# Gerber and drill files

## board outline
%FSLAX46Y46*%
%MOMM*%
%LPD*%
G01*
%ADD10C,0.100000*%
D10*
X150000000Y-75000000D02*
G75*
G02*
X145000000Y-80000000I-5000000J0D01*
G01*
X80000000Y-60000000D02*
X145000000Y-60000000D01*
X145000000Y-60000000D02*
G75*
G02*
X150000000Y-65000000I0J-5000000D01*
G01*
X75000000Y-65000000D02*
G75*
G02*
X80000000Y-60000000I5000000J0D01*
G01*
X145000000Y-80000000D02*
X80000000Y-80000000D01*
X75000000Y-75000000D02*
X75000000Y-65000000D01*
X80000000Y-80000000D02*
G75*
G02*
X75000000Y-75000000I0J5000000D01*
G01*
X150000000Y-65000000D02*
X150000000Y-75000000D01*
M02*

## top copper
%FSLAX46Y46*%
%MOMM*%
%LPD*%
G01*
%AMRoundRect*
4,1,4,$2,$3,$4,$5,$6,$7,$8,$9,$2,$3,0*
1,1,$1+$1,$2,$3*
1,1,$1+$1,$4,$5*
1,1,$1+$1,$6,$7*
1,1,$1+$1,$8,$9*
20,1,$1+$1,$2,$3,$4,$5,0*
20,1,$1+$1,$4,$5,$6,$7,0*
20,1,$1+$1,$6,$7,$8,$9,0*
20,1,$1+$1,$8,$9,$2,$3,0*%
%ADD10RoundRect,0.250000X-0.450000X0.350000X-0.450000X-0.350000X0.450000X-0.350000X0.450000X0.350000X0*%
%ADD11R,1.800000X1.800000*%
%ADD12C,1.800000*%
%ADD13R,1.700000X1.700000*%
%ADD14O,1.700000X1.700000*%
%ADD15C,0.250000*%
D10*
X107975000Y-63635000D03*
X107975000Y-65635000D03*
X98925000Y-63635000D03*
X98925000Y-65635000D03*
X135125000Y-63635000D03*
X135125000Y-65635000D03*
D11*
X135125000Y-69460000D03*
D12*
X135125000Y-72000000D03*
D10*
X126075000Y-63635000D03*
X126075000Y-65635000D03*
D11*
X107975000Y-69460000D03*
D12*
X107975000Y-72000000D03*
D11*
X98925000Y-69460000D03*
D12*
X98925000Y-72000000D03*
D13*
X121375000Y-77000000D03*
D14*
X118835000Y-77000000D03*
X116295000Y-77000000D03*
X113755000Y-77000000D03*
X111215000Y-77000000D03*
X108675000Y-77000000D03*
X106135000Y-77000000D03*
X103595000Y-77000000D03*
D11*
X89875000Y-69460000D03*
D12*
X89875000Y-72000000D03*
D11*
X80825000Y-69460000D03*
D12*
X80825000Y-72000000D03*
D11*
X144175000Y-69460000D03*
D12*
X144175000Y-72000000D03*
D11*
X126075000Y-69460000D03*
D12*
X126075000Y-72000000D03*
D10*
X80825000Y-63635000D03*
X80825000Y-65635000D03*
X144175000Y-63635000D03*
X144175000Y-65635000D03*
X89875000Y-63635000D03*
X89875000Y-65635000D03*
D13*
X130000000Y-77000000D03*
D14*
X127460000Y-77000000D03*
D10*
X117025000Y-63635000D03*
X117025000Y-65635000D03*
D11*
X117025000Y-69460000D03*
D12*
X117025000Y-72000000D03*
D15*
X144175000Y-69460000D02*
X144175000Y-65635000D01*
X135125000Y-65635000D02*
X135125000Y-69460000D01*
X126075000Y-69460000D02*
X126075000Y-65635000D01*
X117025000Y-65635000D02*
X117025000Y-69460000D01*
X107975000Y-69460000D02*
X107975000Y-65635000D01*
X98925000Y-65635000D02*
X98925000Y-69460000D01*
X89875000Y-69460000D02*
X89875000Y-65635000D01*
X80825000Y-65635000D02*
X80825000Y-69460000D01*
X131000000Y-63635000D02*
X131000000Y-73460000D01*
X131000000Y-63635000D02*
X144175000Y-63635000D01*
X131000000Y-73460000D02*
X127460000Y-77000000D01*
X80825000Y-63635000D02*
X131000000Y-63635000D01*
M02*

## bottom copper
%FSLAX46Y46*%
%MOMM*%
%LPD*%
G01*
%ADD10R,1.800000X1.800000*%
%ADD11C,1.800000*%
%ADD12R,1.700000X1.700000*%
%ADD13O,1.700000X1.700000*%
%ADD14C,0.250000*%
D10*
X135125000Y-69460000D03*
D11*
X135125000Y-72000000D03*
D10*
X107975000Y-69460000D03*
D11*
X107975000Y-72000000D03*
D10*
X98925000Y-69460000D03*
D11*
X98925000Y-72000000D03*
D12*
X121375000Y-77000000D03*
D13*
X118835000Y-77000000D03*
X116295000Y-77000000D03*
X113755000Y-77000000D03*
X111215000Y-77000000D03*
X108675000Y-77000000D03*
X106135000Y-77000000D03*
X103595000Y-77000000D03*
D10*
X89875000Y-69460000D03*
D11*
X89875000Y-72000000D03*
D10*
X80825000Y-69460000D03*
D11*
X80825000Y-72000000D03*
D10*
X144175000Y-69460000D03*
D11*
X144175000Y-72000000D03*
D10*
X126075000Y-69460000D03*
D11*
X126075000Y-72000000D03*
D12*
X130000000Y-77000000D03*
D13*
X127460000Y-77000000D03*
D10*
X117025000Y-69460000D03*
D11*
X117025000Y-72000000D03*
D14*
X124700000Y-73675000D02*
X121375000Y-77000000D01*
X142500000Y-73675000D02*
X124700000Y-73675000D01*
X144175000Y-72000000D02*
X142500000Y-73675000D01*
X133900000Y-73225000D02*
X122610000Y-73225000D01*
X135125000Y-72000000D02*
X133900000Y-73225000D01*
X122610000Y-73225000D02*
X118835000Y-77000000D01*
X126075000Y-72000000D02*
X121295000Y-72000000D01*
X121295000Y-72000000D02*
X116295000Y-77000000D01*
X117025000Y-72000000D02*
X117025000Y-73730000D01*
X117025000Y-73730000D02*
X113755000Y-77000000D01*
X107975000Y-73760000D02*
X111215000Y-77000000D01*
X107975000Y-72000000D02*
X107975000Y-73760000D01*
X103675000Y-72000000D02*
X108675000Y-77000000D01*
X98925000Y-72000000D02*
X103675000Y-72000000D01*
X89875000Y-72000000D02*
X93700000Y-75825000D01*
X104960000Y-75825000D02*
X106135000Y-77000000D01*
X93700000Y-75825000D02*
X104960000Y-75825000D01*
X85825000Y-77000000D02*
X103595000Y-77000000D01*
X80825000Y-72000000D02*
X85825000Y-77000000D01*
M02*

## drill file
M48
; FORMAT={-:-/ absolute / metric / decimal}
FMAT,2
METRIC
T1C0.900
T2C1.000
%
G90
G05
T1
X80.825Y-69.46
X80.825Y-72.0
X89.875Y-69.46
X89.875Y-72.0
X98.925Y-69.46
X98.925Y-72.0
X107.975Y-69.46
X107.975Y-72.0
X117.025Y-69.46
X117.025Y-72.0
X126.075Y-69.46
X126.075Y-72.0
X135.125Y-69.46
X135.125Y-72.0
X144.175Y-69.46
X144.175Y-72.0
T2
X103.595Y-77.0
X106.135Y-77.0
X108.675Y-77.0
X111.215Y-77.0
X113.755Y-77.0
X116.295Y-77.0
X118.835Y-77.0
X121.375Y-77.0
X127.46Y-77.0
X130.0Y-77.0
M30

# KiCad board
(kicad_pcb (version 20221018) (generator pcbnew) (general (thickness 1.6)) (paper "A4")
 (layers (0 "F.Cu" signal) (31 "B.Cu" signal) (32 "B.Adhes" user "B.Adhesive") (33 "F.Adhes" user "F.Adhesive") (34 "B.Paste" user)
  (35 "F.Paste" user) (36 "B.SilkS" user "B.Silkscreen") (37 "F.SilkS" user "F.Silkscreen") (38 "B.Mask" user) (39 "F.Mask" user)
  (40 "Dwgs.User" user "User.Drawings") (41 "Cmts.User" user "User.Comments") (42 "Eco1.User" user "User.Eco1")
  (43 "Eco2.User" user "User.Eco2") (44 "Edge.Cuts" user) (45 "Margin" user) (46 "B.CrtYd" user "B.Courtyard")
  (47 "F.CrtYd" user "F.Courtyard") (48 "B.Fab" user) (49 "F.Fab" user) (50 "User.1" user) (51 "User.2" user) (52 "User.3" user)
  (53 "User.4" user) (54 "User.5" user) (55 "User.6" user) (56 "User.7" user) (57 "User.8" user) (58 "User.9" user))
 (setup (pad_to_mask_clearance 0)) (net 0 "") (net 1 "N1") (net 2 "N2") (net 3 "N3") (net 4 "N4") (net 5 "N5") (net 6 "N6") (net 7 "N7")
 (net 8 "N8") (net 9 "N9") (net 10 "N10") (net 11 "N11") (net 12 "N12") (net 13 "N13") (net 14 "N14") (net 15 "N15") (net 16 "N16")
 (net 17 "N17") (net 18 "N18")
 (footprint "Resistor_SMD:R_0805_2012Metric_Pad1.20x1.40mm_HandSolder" (layer "F.Cu") (at 107.975 64.635 -90)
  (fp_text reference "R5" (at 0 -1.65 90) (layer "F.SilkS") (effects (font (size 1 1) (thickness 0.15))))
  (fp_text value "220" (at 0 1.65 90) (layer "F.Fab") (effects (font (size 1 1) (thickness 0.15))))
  (pad "1" smd roundrect (at -1 0 270) (size 1.2 1.4) (layers "F.Cu" "F.Paste" "F.Mask") (roundrect_rratio 0.208333) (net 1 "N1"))
  (pad "2" smd roundrect (at 1 0 270) (size 1.2 1.4) (layers "F.Cu" "F.Paste" "F.Mask") (roundrect_rratio 0.208333) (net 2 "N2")))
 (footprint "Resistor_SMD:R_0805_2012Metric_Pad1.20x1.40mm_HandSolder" (layer "F.Cu") (at 98.925 64.635 -90)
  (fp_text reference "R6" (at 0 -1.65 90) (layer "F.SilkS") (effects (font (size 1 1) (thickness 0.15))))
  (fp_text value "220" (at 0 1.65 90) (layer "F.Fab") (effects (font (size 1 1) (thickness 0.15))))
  (pad "1" smd roundrect (at -1 0 270) (size 1.2 1.4) (layers "F.Cu" "F.Paste" "F.Mask") (roundrect_rratio 0.208333) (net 1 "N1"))
  (pad "2" smd roundrect (at 1 0 270) (size 1.2 1.4) (layers "F.Cu" "F.Paste" "F.Mask") (roundrect_rratio 0.208333) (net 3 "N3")))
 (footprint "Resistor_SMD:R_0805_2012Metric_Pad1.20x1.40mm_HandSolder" (layer "F.Cu") (at 135.125 64.635 -90)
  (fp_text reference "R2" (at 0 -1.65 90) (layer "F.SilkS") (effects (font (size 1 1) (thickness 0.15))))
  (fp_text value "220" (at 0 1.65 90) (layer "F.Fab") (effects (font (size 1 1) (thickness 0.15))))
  (pad "1" smd roundrect (at -1 0 270) (size 1.2 1.4) (layers "F.Cu" "F.Paste" "F.Mask") (roundrect_rratio 0.208333) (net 1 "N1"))
  (pad "2" smd roundrect (at 1 0 270) (size 1.2 1.4) (layers "F.Cu" "F.Paste" "F.Mask") (roundrect_rratio 0.208333) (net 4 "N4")))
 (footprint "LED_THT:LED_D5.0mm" (layer "F.Cu") (at 135.125 69.46 -90)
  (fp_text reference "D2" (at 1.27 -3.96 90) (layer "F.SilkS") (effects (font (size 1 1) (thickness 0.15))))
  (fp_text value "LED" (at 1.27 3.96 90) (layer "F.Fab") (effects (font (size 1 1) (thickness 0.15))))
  (pad "1" thru_hole rect (at 0 0 270) (size 1.8 1.8) (drill 0.9) (layers "*.Cu" "*.Mask") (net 4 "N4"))
  (pad "2" thru_hole circle (at 2.54 0 270) (size 1.8 1.8) (drill 0.9) (layers "*.Cu" "*.Mask") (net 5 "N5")))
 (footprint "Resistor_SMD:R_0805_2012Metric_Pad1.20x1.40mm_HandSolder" (layer "F.Cu") (at 126.075 64.635 -90)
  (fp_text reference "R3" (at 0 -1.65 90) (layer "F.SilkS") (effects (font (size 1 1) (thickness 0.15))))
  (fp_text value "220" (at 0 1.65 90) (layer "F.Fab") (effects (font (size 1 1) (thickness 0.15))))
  (pad "1" smd roundrect (at -1 0 270) (size 1.2 1.4) (layers "F.Cu" "F.Paste" "F.Mask") (roundrect_rratio 0.208333) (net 1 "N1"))
  (pad "2" smd roundrect (at 1 0 270) (size 1.2 1.4) (layers "F.Cu" "F.Paste" "F.Mask") (roundrect_rratio 0.208333) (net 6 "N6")))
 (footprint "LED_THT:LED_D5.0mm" (layer "F.Cu") (at 107.975 69.46 -90)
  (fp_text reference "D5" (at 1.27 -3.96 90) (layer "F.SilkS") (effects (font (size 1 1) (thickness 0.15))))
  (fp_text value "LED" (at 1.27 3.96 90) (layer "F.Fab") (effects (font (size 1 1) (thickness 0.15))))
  (pad "1" thru_hole rect (at 0 0 270) (size 1.8 1.8) (drill 0.9) (layers "*.Cu" "*.Mask") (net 2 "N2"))
  (pad "2" thru_hole circle (at 2.54 0 270) (size 1.8 1.8) (drill 0.9) (layers "*.Cu" "*.Mask") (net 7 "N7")))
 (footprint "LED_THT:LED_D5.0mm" (layer "F.Cu") (at 98.925 69.46 -90)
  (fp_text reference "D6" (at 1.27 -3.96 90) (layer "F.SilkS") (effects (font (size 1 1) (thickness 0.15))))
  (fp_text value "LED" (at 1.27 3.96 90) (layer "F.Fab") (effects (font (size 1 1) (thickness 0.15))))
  (pad "1" thru_hole rect (at 0 0 270) (size 1.8 1.8) (drill 0.9) (layers "*.Cu" "*.Mask") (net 3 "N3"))
  (pad "2" thru_hole circle (at 2.54 0 270) (size 1.8 1.8) (drill 0.9) (layers "*.Cu" "*.Mask") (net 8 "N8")))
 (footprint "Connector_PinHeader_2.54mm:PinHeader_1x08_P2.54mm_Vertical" (layer "F.Cu") (at 121.375 77 -90)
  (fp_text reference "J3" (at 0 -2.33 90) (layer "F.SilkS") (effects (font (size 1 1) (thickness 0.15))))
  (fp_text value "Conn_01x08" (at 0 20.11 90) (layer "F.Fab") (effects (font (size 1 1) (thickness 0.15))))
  (pad "1" thru_hole rect (at 0 0 270) (size 1.7 1.7) (drill 1) (layers "*.Cu" "*.Mask") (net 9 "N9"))
  (pad "2" thru_hole oval (at 0 2.54 270) (size 1.7 1.7) (drill 1) (layers "*.Cu" "*.Mask") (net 5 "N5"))
  (pad "3" thru_hole oval (at 0 5.08 270) (size 1.7 1.7) (drill 1) (layers "*.Cu" "*.Mask") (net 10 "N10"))
  (pad "4" thru_hole oval (at 0 7.62 270) (size 1.7 1.7) (drill 1) (layers "*.Cu" "*.Mask") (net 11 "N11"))
  (pad "5" thru_hole oval (at 0 10.16 270) (size 1.7 1.7) (drill 1) (layers "*.Cu" "*.Mask") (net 7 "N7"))
  (pad "6" thru_hole oval (at 0 12.7 270) (size 1.7 1.7) (drill 1) (layers "*.Cu" "*.Mask") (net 8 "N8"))
  (pad "7" thru_hole oval (at 0 15.24 270) (size 1.7 1.7) (drill 1) (layers "*.Cu" "*.Mask") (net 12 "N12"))
  (pad "8" thru_hole oval (at 0 17.78 270) (size 1.7 1.7) (drill 1) (layers "*.Cu" "*.Mask") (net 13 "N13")))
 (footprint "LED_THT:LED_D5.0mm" (layer "F.Cu") (at 89.875 69.46 -90)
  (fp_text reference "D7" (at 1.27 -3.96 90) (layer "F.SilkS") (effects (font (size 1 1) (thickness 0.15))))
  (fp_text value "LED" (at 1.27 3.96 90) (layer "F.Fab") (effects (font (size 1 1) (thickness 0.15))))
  (pad "1" thru_hole rect (at 0 0 270) (size 1.8 1.8) (drill 0.9) (layers "*.Cu" "*.Mask") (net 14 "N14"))
  (pad "2" thru_hole circle (at 2.54 0 270) (size 1.8 1.8) (drill 0.9) (layers "*.Cu" "*.Mask") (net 12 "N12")))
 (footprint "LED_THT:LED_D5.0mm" (layer "F.Cu") (at 80.825 69.46 -90)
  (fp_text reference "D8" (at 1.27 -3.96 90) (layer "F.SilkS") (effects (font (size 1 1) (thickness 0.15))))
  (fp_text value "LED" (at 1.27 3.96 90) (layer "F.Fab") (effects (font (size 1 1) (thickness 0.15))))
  (pad "1" thru_hole rect (at 0 0 270) (size 1.8 1.8) (drill 0.9) (layers "*.Cu" "*.Mask") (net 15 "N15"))
  (pad "2" thru_hole circle (at 2.54 0 270) (size 1.8 1.8) (drill 0.9) (layers "*.Cu" "*.Mask") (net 13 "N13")))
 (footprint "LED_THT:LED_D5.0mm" (layer "F.Cu") (at 144.175 69.46 -90)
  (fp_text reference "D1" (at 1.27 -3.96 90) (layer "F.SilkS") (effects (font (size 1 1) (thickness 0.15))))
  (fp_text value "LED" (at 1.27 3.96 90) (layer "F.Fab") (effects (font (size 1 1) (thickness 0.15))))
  (pad "1" thru_hole rect (at 0 0 270) (size 1.8 1.8) (drill 0.9) (layers "*.Cu" "*.Mask") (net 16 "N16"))
  (pad "2" thru_hole circle (at 2.54 0 270) (size 1.8 1.8) (drill 0.9) (layers "*.Cu" "*.Mask") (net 9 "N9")))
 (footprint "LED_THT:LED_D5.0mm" (layer "F.Cu") (at 126.075 69.46 -90)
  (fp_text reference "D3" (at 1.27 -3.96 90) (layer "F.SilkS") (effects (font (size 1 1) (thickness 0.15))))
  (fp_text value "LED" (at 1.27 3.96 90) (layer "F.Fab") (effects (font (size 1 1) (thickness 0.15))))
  (pad "1" thru_hole rect (at 0 0 270) (size 1.8 1.8) (drill 0.9) (layers "*.Cu" "*.Mask") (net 6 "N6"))
  (pad "2" thru_hole circle (at 2.54 0 270) (size 1.8 1.8) (drill 0.9) (layers "*.Cu" "*.Mask") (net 10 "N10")))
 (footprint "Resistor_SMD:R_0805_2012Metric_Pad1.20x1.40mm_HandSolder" (layer "F.Cu") (at 80.825 64.635 -90)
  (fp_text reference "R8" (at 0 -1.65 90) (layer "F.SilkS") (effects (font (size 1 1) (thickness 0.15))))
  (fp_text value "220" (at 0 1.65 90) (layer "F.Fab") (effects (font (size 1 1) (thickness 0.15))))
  (pad "1" smd roundrect (at -1 0 270) (size 1.2 1.4) (layers "F.Cu" "F.Paste" "F.Mask") (roundrect_rratio 0.208333) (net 1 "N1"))
  (pad "2" smd roundrect (at 1 0 270) (size 1.2 1.4) (layers "F.Cu" "F.Paste" "F.Mask") (roundrect_rratio 0.208333) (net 15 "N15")))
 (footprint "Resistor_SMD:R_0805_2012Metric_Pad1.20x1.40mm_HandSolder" (layer "F.Cu") (at 144.175 64.635 -90)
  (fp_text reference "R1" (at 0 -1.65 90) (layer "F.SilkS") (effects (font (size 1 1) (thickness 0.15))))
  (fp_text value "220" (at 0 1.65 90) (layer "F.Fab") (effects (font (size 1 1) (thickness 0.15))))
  (pad "1" smd roundrect (at -1 0 270) (size 1.2 1.4) (layers "F.Cu" "F.Paste" "F.Mask") (roundrect_rratio 0.208333) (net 1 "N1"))
  (pad "2" smd roundrect (at 1 0 270) (size 1.2 1.4) (layers "F.Cu" "F.Paste" "F.Mask") (roundrect_rratio 0.208333) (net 16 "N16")))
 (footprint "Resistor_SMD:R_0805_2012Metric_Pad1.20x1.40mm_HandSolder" (layer "F.Cu") (at 89.875 64.635 -90)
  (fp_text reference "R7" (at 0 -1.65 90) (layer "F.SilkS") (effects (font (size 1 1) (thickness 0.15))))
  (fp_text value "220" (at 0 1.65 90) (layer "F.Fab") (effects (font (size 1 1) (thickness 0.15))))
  (pad "1" smd roundrect (at -1 0 270) (size 1.2 1.4) (layers "F.Cu" "F.Paste" "F.Mask") (roundrect_rratio 0.208333) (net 1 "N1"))
  (pad "2" smd roundrect (at 1 0 270) (size 1.2 1.4) (layers "F.Cu" "F.Paste" "F.Mask") (roundrect_rratio 0.208333) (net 14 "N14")))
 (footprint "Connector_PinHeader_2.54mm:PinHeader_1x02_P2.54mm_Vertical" (layer "F.Cu") (at 130 77 -90)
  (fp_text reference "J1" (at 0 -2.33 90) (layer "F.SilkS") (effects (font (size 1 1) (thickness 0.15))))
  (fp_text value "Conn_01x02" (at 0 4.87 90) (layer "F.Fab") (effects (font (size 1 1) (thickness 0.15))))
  (pad "1" thru_hole rect (at 0 0 270) (size 1.7 1.7) (drill 1) (layers "*.Cu" "*.Mask") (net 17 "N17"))
  (pad "2" thru_hole oval (at 0 2.54 270) (size 1.7 1.7) (drill 1) (layers "*.Cu" "*.Mask") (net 1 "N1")))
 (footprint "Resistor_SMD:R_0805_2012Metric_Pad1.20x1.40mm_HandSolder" (layer "F.Cu") (at 117.025 64.635 -90)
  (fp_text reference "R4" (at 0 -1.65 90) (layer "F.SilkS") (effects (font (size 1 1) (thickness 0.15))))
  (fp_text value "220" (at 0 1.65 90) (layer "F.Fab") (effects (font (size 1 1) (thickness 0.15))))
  (pad "1" smd roundrect (at -1 0 270) (size 1.2 1.4) (layers "F.Cu" "F.Paste" "F.Mask") (roundrect_rratio 0.208333) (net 1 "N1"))
  (pad "2" smd roundrect (at 1 0 270) (size 1.2 1.4) (layers "F.Cu" "F.Paste" "F.Mask") (roundrect_rratio 0.208333) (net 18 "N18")))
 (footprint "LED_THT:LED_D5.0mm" (layer "F.Cu") (at 117.025 69.46 -90)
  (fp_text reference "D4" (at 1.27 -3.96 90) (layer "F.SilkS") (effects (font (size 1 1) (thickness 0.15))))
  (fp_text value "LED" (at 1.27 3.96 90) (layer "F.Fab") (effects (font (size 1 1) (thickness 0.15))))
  (pad "1" thru_hole rect (at 0 0 270) (size 1.8 1.8) (drill 0.9) (layers "*.Cu" "*.Mask") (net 18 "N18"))
  (pad "2" thru_hole circle (at 2.54 0 270) (size 1.8 1.8) (drill 0.9) (layers "*.Cu" "*.Mask") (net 11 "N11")))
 (gr_arc (start 150 75) (mid 148.535534 78.535534) (end 145 80) (stroke (width 0.1) (type default)) (layer "Edge.Cuts"))
 (gr_line (start 80 60) (end 145 60) (stroke (width 0.1) (type default)) (layer "Edge.Cuts"))
 (gr_arc (start 145 60) (mid 148.535534 61.464466) (end 150 65) (stroke (width 0.1) (type default)) (layer "Edge.Cuts"))
 (gr_arc (start 75 65) (mid 76.464466 61.464466) (end 80 60) (stroke (width 0.1) (type default)) (layer "Edge.Cuts"))
 (gr_line (start 145 80) (end 80 80) (stroke (width 0.1) (type default)) (layer "Edge.Cuts"))
 (gr_line (start 75 75) (end 75 65) (stroke (width 0.1) (type default)) (layer "Edge.Cuts"))
 (gr_arc (start 80 80) (mid 76.464466 78.535534) (end 75 75) (stroke (width 0.1) (type default)) (layer "Edge.Cuts"))
 (gr_line (start 150 65) (end 150 75) (stroke (width 0.1) (type default)) (layer "Edge.Cuts"))
 (segment (start 144.175 69.46) (end 144.175 65.635) (width 0.25) (layer "F.Cu") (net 16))
 (segment (start 124.7 73.675) (end 121.375 77) (width 0.25) (layer "B.Cu") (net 9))
 (segment (start 142.5 73.675) (end 124.7 73.675) (width 0.25) (layer "B.Cu") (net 9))
 (segment (start 144.175 72) (end 142.5 73.675) (width 0.25) (layer "B.Cu") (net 9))
 (segment (start 135.125 65.635) (end 135.125 69.46) (width 0.25) (layer "F.Cu") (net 4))
 (segment (start 133.9 73.225) (end 122.61 73.225) (width 0.25) (layer "B.Cu") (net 5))
 (segment (start 135.125 72) (end 133.9 73.225) (width 0.25) (layer "B.Cu") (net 5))
 (segment (start 122.61 73.225) (end 118.835 77) (width 0.25) (layer "B.Cu") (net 5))
 (segment (start 126.075 69.46) (end 126.075 65.635) (width 0.25) (layer "F.Cu") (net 6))
 (segment (start 126.075 72) (end 121.295 72) (width 0.25) (layer "B.Cu") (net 10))
 (segment (start 121.295 72) (end 116.295 77) (width 0.25) (layer "B.Cu") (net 10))
 (segment (start 117.025 65.635) (end 117.025 69.46) (width 0.25) (layer "F.Cu") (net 18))
 (segment (start 117.025 72) (end 117.025 73.73) (width 0.25) (layer "B.Cu") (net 11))
 (segment (start 117.025 73.73) (end 113.755 77) (width 0.25) (layer "B.Cu") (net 11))
 (segment (start 107.975 69.46) (end 107.975 65.635) (width 0.25) (layer "F.Cu") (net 2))
 (segment (start 107.975 73.76) (end 111.215 77) (width 0.25) (layer "B.Cu") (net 7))
 (segment (start 107.975 72) (end 107.975 73.76) (width 0.25) (layer "B.Cu") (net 7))
 (segment (start 98.925 65.635) (end 98.925 69.46) (width 0.25) (layer "F.Cu") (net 3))
 (segment (start 103.675 72) (end 108.675 77) (width 0.25) (layer "B.Cu") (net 8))
 (segment (start 98.925 72) (end 103.675 72) (width 0.25) (layer "B.Cu") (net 8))
 (segment (start 89.875 69.46) (end 89.875 65.635) (width 0.25) (layer "F.Cu") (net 14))
 (segment (start 89.875 72) (end 93.7 75.825) (width 0.25) (layer "B.Cu") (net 12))
 (segment (start 104.96 75.825) (end 106.135 77) (width 0.25) (layer "B.Cu") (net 12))
 (segment (start 93.7 75.825) (end 104.96 75.825) (width 0.25) (layer "B.Cu") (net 12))
 (segment (start 80.825 65.635) (end 80.825 69.46) (width 0.25) (layer "F.Cu") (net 15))
 (segment (start 85.825 77) (end 103.595 77) (width 0.25) (layer "B.Cu") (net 13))
 (segment (start 80.825 72) (end 85.825 77) (width 0.25) (layer "B.Cu") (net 13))
 (segment (start 131 63.635) (end 131 73.46) (width 0.25) (layer "F.Cu") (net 1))
 (segment (start 131 63.635) (end 144.175 63.635) (width 0.25) (layer "F.Cu") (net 1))
 (segment (start 131 73.46) (end 127.46 77) (width 0.25) (layer "F.Cu") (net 1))
 (segment (start 80.825 63.635) (end 131 63.635) (width 0.25) (layer "F.Cu") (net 1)))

